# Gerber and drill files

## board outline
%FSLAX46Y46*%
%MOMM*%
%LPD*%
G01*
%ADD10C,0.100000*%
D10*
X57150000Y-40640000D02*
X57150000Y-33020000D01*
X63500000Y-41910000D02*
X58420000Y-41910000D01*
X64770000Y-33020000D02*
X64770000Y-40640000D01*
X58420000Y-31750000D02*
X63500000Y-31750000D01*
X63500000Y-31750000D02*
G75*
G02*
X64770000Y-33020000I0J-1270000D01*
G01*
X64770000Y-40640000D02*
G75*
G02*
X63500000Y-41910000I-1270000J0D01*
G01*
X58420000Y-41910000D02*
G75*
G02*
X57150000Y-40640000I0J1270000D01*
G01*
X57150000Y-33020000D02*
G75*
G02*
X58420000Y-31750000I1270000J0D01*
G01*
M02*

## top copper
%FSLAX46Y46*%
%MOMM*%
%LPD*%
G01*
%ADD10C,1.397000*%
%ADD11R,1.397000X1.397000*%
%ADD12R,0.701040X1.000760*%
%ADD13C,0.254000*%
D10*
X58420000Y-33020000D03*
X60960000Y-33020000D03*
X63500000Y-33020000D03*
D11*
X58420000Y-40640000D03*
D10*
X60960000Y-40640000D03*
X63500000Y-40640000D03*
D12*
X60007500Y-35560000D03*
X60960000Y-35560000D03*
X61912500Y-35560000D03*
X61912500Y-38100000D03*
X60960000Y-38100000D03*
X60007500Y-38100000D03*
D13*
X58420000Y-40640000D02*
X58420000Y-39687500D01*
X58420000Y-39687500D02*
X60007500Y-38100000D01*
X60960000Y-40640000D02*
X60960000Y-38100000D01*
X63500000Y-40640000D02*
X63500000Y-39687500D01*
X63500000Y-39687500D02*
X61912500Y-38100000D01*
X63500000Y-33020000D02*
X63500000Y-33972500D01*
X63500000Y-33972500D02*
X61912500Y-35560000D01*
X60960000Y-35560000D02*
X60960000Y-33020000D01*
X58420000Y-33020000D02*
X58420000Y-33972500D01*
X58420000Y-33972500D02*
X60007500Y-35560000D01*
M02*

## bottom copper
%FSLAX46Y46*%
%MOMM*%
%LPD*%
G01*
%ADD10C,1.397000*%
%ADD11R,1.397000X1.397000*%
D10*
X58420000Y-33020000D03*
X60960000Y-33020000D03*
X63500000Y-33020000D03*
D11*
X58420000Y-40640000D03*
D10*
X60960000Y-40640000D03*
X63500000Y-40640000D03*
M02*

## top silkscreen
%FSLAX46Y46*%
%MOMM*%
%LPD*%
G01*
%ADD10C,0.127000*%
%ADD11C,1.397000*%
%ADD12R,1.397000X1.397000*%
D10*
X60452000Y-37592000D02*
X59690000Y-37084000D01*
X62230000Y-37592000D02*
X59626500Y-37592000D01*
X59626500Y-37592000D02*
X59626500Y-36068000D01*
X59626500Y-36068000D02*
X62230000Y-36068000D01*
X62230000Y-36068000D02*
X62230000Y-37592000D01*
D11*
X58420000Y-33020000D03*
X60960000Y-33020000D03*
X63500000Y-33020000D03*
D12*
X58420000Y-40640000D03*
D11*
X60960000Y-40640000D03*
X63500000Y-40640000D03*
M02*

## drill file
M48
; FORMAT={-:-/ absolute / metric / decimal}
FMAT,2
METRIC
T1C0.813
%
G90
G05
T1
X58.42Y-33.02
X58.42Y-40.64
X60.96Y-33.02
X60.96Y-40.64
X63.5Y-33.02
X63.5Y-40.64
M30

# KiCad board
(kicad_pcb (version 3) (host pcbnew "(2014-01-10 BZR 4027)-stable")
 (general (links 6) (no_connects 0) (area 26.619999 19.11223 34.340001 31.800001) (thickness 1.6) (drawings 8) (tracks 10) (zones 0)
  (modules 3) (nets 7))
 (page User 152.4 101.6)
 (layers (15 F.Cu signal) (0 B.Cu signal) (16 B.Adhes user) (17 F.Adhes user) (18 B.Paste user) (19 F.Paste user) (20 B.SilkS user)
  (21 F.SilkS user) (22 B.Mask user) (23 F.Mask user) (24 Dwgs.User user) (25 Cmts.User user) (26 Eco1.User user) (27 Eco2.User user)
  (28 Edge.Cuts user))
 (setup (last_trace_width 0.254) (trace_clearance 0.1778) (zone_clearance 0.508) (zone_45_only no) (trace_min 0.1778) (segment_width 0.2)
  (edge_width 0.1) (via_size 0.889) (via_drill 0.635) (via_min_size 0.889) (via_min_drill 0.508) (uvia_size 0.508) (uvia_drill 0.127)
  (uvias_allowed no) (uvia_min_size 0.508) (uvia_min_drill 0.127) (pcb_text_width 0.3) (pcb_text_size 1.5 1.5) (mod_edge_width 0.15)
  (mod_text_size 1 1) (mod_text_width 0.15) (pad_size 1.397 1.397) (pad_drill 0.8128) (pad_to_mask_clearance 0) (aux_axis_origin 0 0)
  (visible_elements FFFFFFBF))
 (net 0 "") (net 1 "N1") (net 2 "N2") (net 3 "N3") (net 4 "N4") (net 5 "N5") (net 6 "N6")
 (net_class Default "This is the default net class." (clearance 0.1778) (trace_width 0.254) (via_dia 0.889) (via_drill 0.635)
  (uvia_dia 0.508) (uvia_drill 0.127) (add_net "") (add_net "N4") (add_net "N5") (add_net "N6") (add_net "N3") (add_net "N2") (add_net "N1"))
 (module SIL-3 (layer F.Cu) (at 60.96 33.02)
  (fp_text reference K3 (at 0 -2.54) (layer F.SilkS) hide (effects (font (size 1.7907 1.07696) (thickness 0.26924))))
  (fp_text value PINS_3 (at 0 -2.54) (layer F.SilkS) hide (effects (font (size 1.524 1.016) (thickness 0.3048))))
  (pad 1 thru_hole circle (at -2.54 0) (size 1.397 1.397) (drill 0.8128) (layers *.Cu *.Mask F.SilkS) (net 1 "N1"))
  (pad 2 thru_hole circle (at 0 0) (size 1.397 1.397) (drill 0.8128) (layers *.Cu *.Mask F.SilkS) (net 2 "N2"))
  (pad 3 thru_hole circle (at 2.54 0) (size 1.397 1.397) (drill 0.8128) (layers *.Cu *.Mask F.SilkS) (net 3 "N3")))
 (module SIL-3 (layer F.Cu) (at 60.96 40.64)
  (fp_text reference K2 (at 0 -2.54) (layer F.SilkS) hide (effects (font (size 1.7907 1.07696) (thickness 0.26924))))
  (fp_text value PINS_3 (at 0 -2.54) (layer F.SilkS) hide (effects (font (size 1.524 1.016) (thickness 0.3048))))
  (pad 1 thru_hole rect (at -2.54 0) (size 1.397 1.397) (drill 0.8128) (layers *.Cu *.Mask F.SilkS) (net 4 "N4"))
  (pad 2 thru_hole circle (at 0 0) (size 1.397 1.397) (drill 0.8128) (layers *.Cu *.Mask F.SilkS) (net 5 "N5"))
  (pad 3 thru_hole circle (at 2.54 0) (size 1.397 1.397) (drill 0.8128) (layers *.Cu *.Mask F.SilkS) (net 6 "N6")))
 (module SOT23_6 (layer F.Cu) (at 60.96 36.83)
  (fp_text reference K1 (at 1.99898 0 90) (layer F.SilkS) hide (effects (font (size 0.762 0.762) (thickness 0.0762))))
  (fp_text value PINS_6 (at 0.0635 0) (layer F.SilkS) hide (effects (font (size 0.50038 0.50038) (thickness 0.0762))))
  (fp_line (start -0.508 0.762) (end -1.27 0.254) (layer F.SilkS) (width 0.127))
  (fp_line (start 1.27 0.762) (end -1.3335 0.762) (layer F.SilkS) (width 0.127))
  (fp_line (start -1.3335 0.762) (end -1.3335 -0.762) (layer F.SilkS) (width 0.127))
  (fp_line (start -1.3335 -0.762) (end 1.27 -0.762) (layer F.SilkS) (width 0.127))
  (fp_line (start 1.27 -0.762) (end 1.27 0.762) (layer F.SilkS) (width 0.127))
  (pad 6 smd rect (at -0.9525 -1.27) (size 0.70104 1.00076) (layers F.Cu F.Paste F.Mask) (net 1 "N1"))
  (pad 5 smd rect (at 0 -1.27) (size 0.70104 1.00076) (layers F.Cu F.Paste F.Mask) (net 2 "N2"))
  (pad 4 smd rect (at 0.9525 -1.27) (size 0.70104 1.00076) (layers F.Cu F.Paste F.Mask) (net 3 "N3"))
  (pad 3 smd rect (at 0.9525 1.27) (size 0.70104 1.00076) (layers F.Cu F.Paste F.Mask) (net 6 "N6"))
  (pad 2 smd rect (at 0 1.27) (size 0.70104 1.00076) (layers F.Cu F.Paste F.Mask) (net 5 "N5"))
  (pad 1 smd rect (at -0.9525 1.27) (size 0.70104 1.00076) (layers F.Cu F.Paste F.Mask) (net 4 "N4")))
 (gr_line (start 57.15 40.64) (end 57.15 33.02) (angle 90) (layer Edge.Cuts) (width 0.1))
 (gr_line (start 63.5 41.91) (end 58.42 41.91) (angle 90) (layer Edge.Cuts) (width 0.1))
 (gr_line (start 64.77 33.02) (end 64.77 40.64) (angle 90) (layer Edge.Cuts) (width 0.1))
 (gr_line (start 58.42 31.75) (end 63.5 31.75) (angle 90) (layer Edge.Cuts) (width 0.1))
 (gr_arc (start 63.5 33.02) (end 63.5 31.75) (angle 90) (layer Edge.Cuts) (width 0.1))
 (gr_arc (start 63.5 40.64) (end 64.77 40.64) (angle 90) (layer Edge.Cuts) (width 0.1))
 (gr_arc (start 58.42 40.64) (end 58.42 41.91) (angle 90) (layer Edge.Cuts) (width 0.1))
 (gr_arc (start 58.42 33.02) (end 57.15 33.02) (angle 90) (layer Edge.Cuts) (width 0.1))
 (segment (start 58.42 40.64) (end 58.42 39.6875) (width 0.254) (layer F.Cu) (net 4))
 (segment (start 58.42 39.6875) (end 60.0075 38.1) (width 0.254) (layer F.Cu) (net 4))
 (segment (start 60.96 40.64) (end 60.96 38.1) (width 0.254) (layer F.Cu) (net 5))
 (segment (start 63.5 40.64) (end 63.5 39.6875) (width 0.254) (layer F.Cu) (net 6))
 (segment (start 63.5 39.6875) (end 61.9125 38.1) (width 0.254) (layer F.Cu) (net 6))
 (segment (start 63.5 33.02) (end 63.5 33.9725) (width 0.254) (layer F.Cu) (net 3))
 (segment (start 63.5 33.9725) (end 61.9125 35.56) (width 0.254) (layer F.Cu) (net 3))
 (segment (start 60.96 35.56) (end 60.96 33.02) (width 0.254) (layer F.Cu) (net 2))
 (segment (start 58.42 33.02) (end 58.42 33.9725) (width 0.254) (layer F.Cu) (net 1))
 (segment (start 58.42 33.9725) (end 60.0075 35.56) (width 0.254) (layer F.Cu) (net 1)))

